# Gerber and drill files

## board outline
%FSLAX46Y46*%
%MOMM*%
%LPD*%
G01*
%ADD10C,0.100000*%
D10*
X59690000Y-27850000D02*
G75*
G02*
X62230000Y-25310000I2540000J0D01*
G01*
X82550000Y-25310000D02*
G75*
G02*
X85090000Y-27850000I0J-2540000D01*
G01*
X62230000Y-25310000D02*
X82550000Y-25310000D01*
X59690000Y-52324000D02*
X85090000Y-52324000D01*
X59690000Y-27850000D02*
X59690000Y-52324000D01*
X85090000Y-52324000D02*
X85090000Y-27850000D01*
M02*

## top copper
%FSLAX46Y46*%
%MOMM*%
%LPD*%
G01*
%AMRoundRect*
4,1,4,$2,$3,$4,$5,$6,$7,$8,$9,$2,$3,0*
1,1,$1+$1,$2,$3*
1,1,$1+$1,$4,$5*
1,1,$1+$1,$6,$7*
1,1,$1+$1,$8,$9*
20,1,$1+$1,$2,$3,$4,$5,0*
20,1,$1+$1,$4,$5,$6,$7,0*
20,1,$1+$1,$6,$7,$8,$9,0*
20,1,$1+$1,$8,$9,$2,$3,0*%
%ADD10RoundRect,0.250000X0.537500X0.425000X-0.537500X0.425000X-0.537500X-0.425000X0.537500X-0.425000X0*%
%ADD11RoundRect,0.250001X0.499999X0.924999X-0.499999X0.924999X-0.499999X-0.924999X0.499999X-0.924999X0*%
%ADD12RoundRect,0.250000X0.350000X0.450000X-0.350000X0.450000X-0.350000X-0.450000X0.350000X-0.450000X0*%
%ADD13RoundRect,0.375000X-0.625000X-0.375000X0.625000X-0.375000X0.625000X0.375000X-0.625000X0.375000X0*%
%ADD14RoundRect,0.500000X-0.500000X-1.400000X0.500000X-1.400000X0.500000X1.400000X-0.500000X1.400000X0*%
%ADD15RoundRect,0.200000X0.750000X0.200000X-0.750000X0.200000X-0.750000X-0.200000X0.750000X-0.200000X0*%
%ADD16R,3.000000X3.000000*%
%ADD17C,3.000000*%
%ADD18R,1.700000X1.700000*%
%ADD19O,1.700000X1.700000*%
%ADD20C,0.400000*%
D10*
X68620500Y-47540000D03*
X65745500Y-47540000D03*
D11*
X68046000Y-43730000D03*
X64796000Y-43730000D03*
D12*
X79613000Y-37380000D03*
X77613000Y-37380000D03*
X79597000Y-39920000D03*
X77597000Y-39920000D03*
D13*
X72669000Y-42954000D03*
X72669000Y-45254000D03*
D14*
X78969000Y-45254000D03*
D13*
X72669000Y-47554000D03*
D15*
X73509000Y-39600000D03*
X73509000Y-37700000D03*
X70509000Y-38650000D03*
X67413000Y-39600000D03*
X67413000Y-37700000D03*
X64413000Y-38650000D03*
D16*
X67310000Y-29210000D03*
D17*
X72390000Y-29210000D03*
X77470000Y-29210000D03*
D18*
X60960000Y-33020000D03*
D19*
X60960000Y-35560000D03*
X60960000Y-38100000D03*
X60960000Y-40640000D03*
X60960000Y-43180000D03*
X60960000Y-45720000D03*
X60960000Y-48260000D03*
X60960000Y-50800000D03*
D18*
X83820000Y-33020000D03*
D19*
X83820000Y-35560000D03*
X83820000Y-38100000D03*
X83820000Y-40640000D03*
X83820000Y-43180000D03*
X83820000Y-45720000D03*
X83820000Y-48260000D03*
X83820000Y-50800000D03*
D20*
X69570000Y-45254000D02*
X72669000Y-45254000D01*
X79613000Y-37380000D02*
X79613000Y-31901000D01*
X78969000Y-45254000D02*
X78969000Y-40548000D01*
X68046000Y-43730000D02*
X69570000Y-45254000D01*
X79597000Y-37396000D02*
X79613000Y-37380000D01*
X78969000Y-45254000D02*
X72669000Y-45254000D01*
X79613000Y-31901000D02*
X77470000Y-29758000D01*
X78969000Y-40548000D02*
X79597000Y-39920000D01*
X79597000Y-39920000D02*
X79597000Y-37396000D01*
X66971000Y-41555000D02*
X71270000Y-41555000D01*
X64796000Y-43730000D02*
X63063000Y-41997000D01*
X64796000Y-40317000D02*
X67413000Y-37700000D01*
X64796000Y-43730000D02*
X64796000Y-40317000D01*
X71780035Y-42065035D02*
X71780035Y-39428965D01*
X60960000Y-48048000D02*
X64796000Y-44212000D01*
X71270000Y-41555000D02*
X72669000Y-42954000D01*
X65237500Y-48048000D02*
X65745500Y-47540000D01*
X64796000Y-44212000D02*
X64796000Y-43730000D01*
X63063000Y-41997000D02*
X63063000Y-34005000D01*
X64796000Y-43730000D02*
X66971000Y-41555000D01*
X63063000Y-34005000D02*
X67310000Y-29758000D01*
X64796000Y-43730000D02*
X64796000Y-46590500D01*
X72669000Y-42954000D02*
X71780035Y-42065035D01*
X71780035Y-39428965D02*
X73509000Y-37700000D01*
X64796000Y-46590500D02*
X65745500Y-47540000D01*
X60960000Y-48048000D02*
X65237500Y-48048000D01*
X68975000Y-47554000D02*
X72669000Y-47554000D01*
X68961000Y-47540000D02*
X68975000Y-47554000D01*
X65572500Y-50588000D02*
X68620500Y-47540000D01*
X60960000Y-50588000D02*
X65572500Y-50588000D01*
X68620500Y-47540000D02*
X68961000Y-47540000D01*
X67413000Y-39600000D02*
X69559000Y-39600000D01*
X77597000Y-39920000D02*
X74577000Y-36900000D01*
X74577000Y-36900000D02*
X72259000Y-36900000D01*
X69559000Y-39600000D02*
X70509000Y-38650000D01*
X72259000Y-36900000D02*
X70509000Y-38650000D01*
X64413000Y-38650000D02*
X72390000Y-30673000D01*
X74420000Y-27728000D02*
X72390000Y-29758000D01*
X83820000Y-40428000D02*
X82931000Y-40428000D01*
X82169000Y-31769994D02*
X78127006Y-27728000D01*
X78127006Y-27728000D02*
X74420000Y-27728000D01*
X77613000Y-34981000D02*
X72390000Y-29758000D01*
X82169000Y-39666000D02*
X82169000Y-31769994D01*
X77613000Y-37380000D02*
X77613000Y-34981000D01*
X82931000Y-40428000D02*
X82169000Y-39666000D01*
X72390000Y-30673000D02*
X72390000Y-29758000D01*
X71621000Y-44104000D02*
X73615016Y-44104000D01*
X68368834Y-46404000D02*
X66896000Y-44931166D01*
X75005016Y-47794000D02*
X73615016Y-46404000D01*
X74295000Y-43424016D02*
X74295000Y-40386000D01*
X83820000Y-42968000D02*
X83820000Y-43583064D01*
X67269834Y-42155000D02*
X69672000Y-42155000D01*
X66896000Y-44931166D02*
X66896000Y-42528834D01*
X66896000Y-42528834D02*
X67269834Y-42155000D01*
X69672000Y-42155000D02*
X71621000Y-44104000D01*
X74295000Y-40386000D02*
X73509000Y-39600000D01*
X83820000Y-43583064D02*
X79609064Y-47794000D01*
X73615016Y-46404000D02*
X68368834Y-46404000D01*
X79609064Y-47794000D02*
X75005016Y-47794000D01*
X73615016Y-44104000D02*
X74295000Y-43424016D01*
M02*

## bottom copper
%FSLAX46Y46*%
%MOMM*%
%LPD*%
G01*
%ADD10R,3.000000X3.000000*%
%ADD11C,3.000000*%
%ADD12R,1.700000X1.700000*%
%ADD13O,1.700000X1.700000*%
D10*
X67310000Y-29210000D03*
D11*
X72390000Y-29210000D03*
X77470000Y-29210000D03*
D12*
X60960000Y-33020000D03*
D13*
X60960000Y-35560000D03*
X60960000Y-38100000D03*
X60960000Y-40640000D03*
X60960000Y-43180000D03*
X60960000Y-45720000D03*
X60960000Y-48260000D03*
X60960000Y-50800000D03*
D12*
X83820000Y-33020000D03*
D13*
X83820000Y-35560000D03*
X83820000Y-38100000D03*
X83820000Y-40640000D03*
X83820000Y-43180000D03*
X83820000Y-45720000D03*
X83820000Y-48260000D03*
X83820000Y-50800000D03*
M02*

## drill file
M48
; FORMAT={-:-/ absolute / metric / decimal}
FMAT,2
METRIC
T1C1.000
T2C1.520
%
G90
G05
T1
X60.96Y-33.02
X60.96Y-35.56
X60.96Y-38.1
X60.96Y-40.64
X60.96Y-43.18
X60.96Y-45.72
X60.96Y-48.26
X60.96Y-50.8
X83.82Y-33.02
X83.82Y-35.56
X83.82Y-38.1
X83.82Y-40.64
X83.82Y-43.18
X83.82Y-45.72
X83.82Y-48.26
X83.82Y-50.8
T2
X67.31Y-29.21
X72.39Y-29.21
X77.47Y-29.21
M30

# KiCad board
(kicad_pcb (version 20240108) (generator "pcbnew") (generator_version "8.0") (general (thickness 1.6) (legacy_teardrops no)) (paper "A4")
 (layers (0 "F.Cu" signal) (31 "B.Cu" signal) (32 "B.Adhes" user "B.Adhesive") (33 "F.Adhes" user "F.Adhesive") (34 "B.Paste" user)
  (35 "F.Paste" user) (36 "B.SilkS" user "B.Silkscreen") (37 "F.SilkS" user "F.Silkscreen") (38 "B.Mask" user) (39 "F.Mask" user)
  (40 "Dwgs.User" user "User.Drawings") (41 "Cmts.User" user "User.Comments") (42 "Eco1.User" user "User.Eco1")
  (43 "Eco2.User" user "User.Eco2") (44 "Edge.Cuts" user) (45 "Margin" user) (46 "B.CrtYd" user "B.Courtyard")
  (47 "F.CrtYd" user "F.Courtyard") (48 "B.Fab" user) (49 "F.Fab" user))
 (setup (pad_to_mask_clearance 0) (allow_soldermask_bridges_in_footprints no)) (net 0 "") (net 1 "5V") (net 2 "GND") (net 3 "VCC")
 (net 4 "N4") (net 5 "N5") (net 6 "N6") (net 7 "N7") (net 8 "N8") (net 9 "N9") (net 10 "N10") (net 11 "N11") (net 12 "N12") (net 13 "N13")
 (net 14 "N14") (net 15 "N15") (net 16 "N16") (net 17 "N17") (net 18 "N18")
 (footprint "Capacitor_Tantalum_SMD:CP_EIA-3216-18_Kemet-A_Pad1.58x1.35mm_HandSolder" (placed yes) (layer "F.Cu") (at 67.183 47.54 180)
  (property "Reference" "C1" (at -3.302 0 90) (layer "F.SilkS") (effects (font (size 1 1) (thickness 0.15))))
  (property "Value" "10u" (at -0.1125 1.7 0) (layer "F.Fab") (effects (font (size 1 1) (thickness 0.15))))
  (pad "1" smd roundrect (at -1.4375 0 180) (size 1.575 1.35) (layers "F.Cu" "F.Paste" "F.Mask") (roundrect_rratio 0.185185) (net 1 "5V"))
  (pad "2" smd roundrect (at 1.4375 0 180) (size 1.575 1.35) (layers "F.Cu" "F.Paste" "F.Mask") (roundrect_rratio 0.185185) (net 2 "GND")))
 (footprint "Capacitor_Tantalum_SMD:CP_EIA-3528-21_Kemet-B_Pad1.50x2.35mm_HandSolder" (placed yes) (layer "F.Cu") (at 66.421 43.73 180)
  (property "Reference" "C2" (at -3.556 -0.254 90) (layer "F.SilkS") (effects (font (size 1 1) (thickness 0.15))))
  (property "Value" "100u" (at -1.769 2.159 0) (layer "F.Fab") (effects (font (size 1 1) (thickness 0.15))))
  (pad "1" smd roundrect (at -1.625 0 180) (size 1.5 2.35) (layers "F.Cu" "F.Paste" "F.Mask") (roundrect_rratio 0.166667) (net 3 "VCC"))
  (pad "2" smd roundrect (at 1.625 0 180) (size 1.5 2.35) (layers "F.Cu" "F.Paste" "F.Mask") (roundrect_rratio 0.166667) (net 2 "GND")))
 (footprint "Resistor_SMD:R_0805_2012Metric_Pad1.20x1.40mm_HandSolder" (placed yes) (layer "F.Cu") (at 78.613 37.38 180)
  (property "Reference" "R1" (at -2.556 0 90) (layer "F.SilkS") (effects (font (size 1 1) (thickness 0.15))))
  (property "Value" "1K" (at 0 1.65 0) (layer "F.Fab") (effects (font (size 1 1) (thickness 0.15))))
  (pad "1" smd roundrect (at -1 0 180) (size 1.2 1.4) (layers "F.Cu" "F.Paste" "F.Mask") (roundrect_rratio 0.208333) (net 3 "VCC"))
  (pad "2" smd roundrect (at 1 0 180) (size 1.2 1.4) (layers "F.Cu" "F.Paste" "F.Mask") (roundrect_rratio 0.208333) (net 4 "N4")))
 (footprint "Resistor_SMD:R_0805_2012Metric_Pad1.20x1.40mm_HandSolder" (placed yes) (layer "F.Cu") (at 78.597 39.92 180)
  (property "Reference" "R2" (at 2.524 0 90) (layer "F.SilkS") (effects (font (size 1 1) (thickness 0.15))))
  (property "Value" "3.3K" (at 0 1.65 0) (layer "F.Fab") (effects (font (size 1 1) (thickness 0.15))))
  (pad "1" smd roundrect (at -1 0 180) (size 1.2 1.4) (layers "F.Cu" "F.Paste" "F.Mask") (roundrect_rratio 0.208333) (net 3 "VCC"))
  (pad "2" smd roundrect (at 1 0 180) (size 1.2 1.4) (layers "F.Cu" "F.Paste" "F.Mask") (roundrect_rratio 0.208333) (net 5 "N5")))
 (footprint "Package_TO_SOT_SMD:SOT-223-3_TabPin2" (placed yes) (layer "F.Cu") (at 75.819 45.254)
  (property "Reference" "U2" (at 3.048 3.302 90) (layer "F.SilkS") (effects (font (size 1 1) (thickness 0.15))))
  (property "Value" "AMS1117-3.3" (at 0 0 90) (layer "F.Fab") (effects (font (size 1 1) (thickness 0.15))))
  (pad "1" smd roundrect (at -3.15 -2.3) (size 2 1.5) (layers "F.Cu" "F.Paste" "F.Mask") (roundrect_rratio 0.25) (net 2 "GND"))
  (pad "2" smd roundrect (at -3.15 0) (size 2 1.5) (layers "F.Cu" "F.Paste" "F.Mask") (roundrect_rratio 0.25) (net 3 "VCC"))
  (pad "2" smd roundrect (at 3.15 0) (size 2 3.8) (layers "F.Cu" "F.Paste" "F.Mask") (roundrect_rratio 0.25) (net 3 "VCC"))
  (pad "3" smd roundrect (at -3.15 2.3) (size 2 1.5) (layers "F.Cu" "F.Paste" "F.Mask") (roundrect_rratio 0.25) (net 1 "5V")))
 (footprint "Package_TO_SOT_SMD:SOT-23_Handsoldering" (layer "F.Cu") (at 72.009 38.65 180)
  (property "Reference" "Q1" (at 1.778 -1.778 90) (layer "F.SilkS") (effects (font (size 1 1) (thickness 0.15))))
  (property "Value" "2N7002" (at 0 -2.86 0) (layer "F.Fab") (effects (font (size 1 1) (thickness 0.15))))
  (pad "1" smd roundrect (at -1.5 -0.95 180) (size 1.9 0.8) (layers "F.Cu" "F.Paste" "F.Mask") (roundrect_rratio 0.25) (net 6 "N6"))
  (pad "2" smd roundrect (at -1.5 0.95 180) (size 1.9 0.8) (layers "F.Cu" "F.Paste" "F.Mask") (roundrect_rratio 0.25) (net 2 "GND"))
  (pad "3" smd roundrect (at 1.5 0 180) (size 1.9 0.8) (layers "F.Cu" "F.Paste" "F.Mask") (roundrect_rratio 0.25) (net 5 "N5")))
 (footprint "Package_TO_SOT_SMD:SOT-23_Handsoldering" (layer "F.Cu") (at 65.913 38.65 180)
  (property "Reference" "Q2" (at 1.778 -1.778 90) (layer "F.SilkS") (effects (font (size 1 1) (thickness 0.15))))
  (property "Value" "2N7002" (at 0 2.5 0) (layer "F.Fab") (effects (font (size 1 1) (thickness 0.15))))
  (pad "1" smd roundrect (at -1.5 -0.95 180) (size 1.9 0.8) (layers "F.Cu" "F.Paste" "F.Mask") (roundrect_rratio 0.25) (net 5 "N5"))
  (pad "2" smd roundrect (at -1.5 0.95 180) (size 1.9 0.8) (layers "F.Cu" "F.Paste" "F.Mask") (roundrect_rratio 0.25) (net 2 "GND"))
  (pad "3" smd roundrect (at 1.5 0 180) (size 1.9 0.8) (layers "F.Cu" "F.Paste" "F.Mask") (roundrect_rratio 0.25) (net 4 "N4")))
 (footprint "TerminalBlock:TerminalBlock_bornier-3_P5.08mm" (layer "F.Cu") (at 67.31 29.21)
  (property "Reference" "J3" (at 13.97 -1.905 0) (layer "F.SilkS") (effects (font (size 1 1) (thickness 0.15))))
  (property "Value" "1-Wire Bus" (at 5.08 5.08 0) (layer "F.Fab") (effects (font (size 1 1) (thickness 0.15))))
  (pad "1" thru_hole rect (at 0 0) (size 3 3) (drill 1.52) (layers "*.Cu" "*.Mask") (remove_unused_layers no) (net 2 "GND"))
  (pad "2" thru_hole circle (at 5.08 0) (size 3 3) (drill 1.52) (layers "*.Cu" "*.Mask") (remove_unused_layers no) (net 4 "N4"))
  (pad "3" thru_hole circle (at 10.16 0) (size 3 3) (drill 1.52) (layers "*.Cu" "*.Mask") (remove_unused_layers no) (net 3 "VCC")))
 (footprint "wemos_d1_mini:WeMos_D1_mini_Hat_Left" (layer "B.Cu") (at 60.96 33.02 180)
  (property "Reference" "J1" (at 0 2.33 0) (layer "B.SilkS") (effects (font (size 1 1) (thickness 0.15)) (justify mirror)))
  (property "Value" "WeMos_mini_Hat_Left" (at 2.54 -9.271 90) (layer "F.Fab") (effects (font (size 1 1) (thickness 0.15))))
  (pad "1" thru_hole rect (at 0 0 180) (size 1.7 1.7) (drill 1) (layers "*.Cu" "*.Mask") (remove_unused_layers no) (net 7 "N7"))
  (pad "2" thru_hole oval (at 0 -2.54 180) (size 1.7 1.7) (drill 1) (layers "*.Cu" "*.Mask") (remove_unused_layers no) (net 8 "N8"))
  (pad "3" thru_hole oval (at 0 -5.08 180) (size 1.7 1.7) (drill 1) (layers "*.Cu" "*.Mask") (remove_unused_layers no) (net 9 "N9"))
  (pad "4" thru_hole oval (at 0 -7.62 180) (size 1.7 1.7) (drill 1) (layers "*.Cu" "*.Mask") (remove_unused_layers no) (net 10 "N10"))
  (pad "5" thru_hole oval (at 0 -10.16 180) (size 1.7 1.7) (drill 1) (layers "*.Cu" "*.Mask") (remove_unused_layers no) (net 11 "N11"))
  (pad "6" thru_hole oval (at 0 -12.7 180) (size 1.7 1.7) (drill 1) (layers "*.Cu" "*.Mask") (remove_unused_layers no) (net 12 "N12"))
  (pad "7" thru_hole oval (at 0 -15.24 180) (size 1.7 1.7) (drill 1) (layers "*.Cu" "*.Mask") (remove_unused_layers no) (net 2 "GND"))
  (pad "8" thru_hole oval (at 0 -17.78 180) (size 1.7 1.7) (drill 1) (layers "*.Cu" "*.Mask") (remove_unused_layers no) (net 1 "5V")))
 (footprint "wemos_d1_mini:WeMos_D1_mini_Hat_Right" (layer "B.Cu") (at 83.82 33.02 180)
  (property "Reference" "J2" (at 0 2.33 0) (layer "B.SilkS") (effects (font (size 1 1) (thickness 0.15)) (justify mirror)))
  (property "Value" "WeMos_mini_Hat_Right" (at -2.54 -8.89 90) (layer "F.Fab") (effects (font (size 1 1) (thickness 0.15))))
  (pad "1" thru_hole rect (at 0 0 180) (size 1.7 1.7) (drill 1) (layers "*.Cu" "*.Mask") (remove_unused_layers no) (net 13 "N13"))
  (pad "2" thru_hole oval (at 0 -2.54 180) (size 1.7 1.7) (drill 1) (layers "*.Cu" "*.Mask") (remove_unused_layers no) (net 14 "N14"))
  (pad "3" thru_hole oval (at 0 -5.08 180) (size 1.7 1.7) (drill 1) (layers "*.Cu" "*.Mask") (remove_unused_layers no) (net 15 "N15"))
  (pad "4" thru_hole oval (at 0 -7.62 180) (size 1.7 1.7) (drill 1) (layers "*.Cu" "*.Mask") (remove_unused_layers no) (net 4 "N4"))
  (pad "5" thru_hole oval (at 0 -10.16 180) (size 1.7 1.7) (drill 1) (layers "*.Cu" "*.Mask") (remove_unused_layers no) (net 6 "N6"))
  (pad "6" thru_hole oval (at 0 -12.7 180) (size 1.7 1.7) (drill 1) (layers "*.Cu" "*.Mask") (remove_unused_layers no) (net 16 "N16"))
  (pad "7" thru_hole oval (at 0 -15.24 180) (size 1.7 1.7) (drill 1) (layers "*.Cu" "*.Mask") (remove_unused_layers no) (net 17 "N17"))
  (pad "8" thru_hole oval (at 0 -17.78 180) (size 1.7 1.7) (drill 1) (layers "*.Cu" "*.Mask") (remove_unused_layers no) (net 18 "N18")))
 (gr_arc (start 59.69 27.85) (mid 60.433949 26.053949) (end 62.23 25.31) (stroke (width 0.1) (type default)) (layer "Edge.Cuts"))
 (gr_arc (start 82.55 25.31) (mid 84.346051 26.053949) (end 85.09 27.85) (stroke (width 0.1) (type default)) (layer "Edge.Cuts"))
 (gr_line (start 62.23 25.31) (end 82.55 25.31) (stroke (width 0.1) (type default)) (layer "Edge.Cuts"))
 (gr_line (start 59.69 52.324) (end 85.09 52.324) (stroke (width 0.1) (type default)) (layer "Edge.Cuts"))
 (gr_line (start 59.69 27.85) (end 59.69 52.324) (stroke (width 0.1) (type default)) (layer "Edge.Cuts"))
 (gr_line (start 85.09 52.324) (end 85.09 27.85) (stroke (width 0.1) (type default)) (layer "Edge.Cuts"))
 (segment (start 69.57 45.254) (end 72.669 45.254) (width 0.4) (layer "F.Cu") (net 3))
 (segment (start 79.613 37.38) (end 79.613 31.901) (width 0.4) (layer "F.Cu") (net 3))
 (segment (start 78.969 45.254) (end 78.969 40.548) (width 0.4) (layer "F.Cu") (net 3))
 (segment (start 68.046 43.73) (end 69.57 45.254) (width 0.4) (layer "F.Cu") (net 3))
 (segment (start 79.597 37.396) (end 79.613 37.38) (width 0.4) (layer "F.Cu") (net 3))
 (segment (start 78.969 45.254) (end 72.669 45.254) (width 0.4) (layer "F.Cu") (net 3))
 (segment (start 79.613 31.901) (end 77.47 29.758) (width 0.4) (layer "F.Cu") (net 3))
 (segment (start 78.969 40.548) (end 79.597 39.92) (width 0.4) (layer "F.Cu") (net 3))
 (segment (start 79.597 39.92) (end 79.597 37.396) (width 0.4) (layer "F.Cu") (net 3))
 (segment (start 66.971 41.555) (end 71.27 41.555) (width 0.4) (layer "F.Cu") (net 2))
 (segment (start 64.796 43.73) (end 63.063 41.997) (width 0.4) (layer "F.Cu") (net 2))
 (segment (start 64.796 40.317) (end 67.413 37.7) (width 0.4) (layer "F.Cu") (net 2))
 (segment (start 64.796 43.73) (end 64.796 40.317) (width 0.4) (layer "F.Cu") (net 2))
 (segment (start 71.780035 42.065035) (end 71.780035 39.428965) (width 0.4) (layer "F.Cu") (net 2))
 (segment (start 60.96 48.048) (end 64.796 44.212) (width 0.4) (layer "F.Cu") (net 2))
 (segment (start 71.27 41.555) (end 72.669 42.954) (width 0.4) (layer "F.Cu") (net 2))
 (segment (start 65.2375 48.048) (end 65.7455 47.54) (width 0.4) (layer "F.Cu") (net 2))
 (segment (start 64.796 44.212) (end 64.796 43.73) (width 0.4) (layer "F.Cu") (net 2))
 (segment (start 63.063 41.997) (end 63.063 34.005) (width 0.4) (layer "F.Cu") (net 2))
 (segment (start 64.796 43.73) (end 66.971 41.555) (width 0.4) (layer "F.Cu") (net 2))
 (segment (start 63.063 34.005) (end 67.31 29.758) (width 0.4) (layer "F.Cu") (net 2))
 (segment (start 64.796 43.73) (end 64.796 46.5905) (width 0.4) (layer "F.Cu") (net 2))
 (segment (start 72.669 42.954) (end 71.780035 42.065035) (width 0.4) (layer "F.Cu") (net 2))
 (segment (start 71.780035 39.428965) (end 73.509 37.7) (width 0.4) (layer "F.Cu") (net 2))
 (segment (start 64.796 46.5905) (end 65.7455 47.54) (width 0.4) (layer "F.Cu") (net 2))
 (segment (start 60.96 48.048) (end 65.2375 48.048) (width 0.4) (layer "F.Cu") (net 2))
 (segment (start 68.975 47.554) (end 72.669 47.554) (width 0.4) (layer "F.Cu") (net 1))
 (segment (start 68.961 47.54) (end 68.975 47.554) (width 0.4) (layer "F.Cu") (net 1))
 (segment (start 65.5725 50.588) (end 68.6205 47.54) (width 0.4) (layer "F.Cu") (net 1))
 (segment (start 60.96 50.588) (end 65.5725 50.588) (width 0.4) (layer "F.Cu") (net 1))
 (segment (start 68.6205 47.54) (end 68.961 47.54) (width 0.4) (layer "F.Cu") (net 1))
 (segment (start 67.413 39.6) (end 69.559 39.6) (width 0.4) (layer "F.Cu") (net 5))
 (segment (start 77.597 39.92) (end 74.577 36.9) (width 0.4) (layer "F.Cu") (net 5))
 (segment (start 74.577 36.9) (end 72.259 36.9) (width 0.4) (layer "F.Cu") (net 5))
 (segment (start 69.559 39.6) (end 70.509 38.65) (width 0.4) (layer "F.Cu") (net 5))
 (segment (start 72.259 36.9) (end 70.509 38.65) (width 0.4) (layer "F.Cu") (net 5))
 (segment (start 64.413 38.65) (end 72.39 30.673) (width 0.4) (layer "F.Cu") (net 4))
 (segment (start 74.42 27.728) (end 72.39 29.758) (width 0.4) (layer "F.Cu") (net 4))
 (segment (start 83.82 40.428) (end 82.931 40.428) (width 0.4) (layer "F.Cu") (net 4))
 (segment (start 82.169 31.769994) (end 78.127006 27.728) (width 0.4) (layer "F.Cu") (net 4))
 (segment (start 78.127006 27.728) (end 74.42 27.728) (width 0.4) (layer "F.Cu") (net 4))
 (segment (start 77.613 34.981) (end 72.39 29.758) (width 0.4) (layer "F.Cu") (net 4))
 (segment (start 82.169 39.666) (end 82.169 31.769994) (width 0.4) (layer "F.Cu") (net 4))
 (segment (start 77.613 37.38) (end 77.613 34.981) (width 0.4) (layer "F.Cu") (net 4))
 (segment (start 82.931 40.428) (end 82.169 39.666) (width 0.4) (layer "F.Cu") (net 4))
 (segment (start 72.39 30.673) (end 72.39 29.758) (width 0.4) (layer "F.Cu") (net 4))
 (segment (start 71.621 44.104) (end 73.615016 44.104) (width 0.4) (layer "F.Cu") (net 6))
 (segment (start 68.368834 46.404) (end 66.896 44.931166) (width 0.4) (layer "F.Cu") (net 6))
 (segment (start 75.005016 47.794) (end 73.615016 46.404) (width 0.4) (layer "F.Cu") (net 6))
 (segment (start 74.295 43.424016) (end 74.295 40.386) (width 0.4) (layer "F.Cu") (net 6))
 (segment (start 83.82 42.968) (end 83.82 43.583064) (width 0.4) (layer "F.Cu") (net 6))
 (segment (start 67.269834 42.155) (end 69.672 42.155) (width 0.4) (layer "F.Cu") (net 6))
 (segment (start 66.896 44.931166) (end 66.896 42.528834) (width 0.4) (layer "F.Cu") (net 6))
 (segment (start 66.896 42.528834) (end 67.269834 42.155) (width 0.4) (layer "F.Cu") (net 6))
 (segment (start 69.672 42.155) (end 71.621 44.104) (width 0.4) (layer "F.Cu") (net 6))
 (segment (start 74.295 40.386) (end 73.509 39.6) (width 0.4) (layer "F.Cu") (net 6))
 (segment (start 83.82 43.583064) (end 79.609064 47.794) (width 0.4) (layer "F.Cu") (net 6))
 (segment (start 73.615016 46.404) (end 68.368834 46.404) (width 0.4) (layer "F.Cu") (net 6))
 (segment (start 79.609064 47.794) (end 75.005016 47.794) (width 0.4) (layer "F.Cu") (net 6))
 (segment (start 73.615016 44.104) (end 74.295 43.424016) (width 0.4) (layer "F.Cu") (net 6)))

